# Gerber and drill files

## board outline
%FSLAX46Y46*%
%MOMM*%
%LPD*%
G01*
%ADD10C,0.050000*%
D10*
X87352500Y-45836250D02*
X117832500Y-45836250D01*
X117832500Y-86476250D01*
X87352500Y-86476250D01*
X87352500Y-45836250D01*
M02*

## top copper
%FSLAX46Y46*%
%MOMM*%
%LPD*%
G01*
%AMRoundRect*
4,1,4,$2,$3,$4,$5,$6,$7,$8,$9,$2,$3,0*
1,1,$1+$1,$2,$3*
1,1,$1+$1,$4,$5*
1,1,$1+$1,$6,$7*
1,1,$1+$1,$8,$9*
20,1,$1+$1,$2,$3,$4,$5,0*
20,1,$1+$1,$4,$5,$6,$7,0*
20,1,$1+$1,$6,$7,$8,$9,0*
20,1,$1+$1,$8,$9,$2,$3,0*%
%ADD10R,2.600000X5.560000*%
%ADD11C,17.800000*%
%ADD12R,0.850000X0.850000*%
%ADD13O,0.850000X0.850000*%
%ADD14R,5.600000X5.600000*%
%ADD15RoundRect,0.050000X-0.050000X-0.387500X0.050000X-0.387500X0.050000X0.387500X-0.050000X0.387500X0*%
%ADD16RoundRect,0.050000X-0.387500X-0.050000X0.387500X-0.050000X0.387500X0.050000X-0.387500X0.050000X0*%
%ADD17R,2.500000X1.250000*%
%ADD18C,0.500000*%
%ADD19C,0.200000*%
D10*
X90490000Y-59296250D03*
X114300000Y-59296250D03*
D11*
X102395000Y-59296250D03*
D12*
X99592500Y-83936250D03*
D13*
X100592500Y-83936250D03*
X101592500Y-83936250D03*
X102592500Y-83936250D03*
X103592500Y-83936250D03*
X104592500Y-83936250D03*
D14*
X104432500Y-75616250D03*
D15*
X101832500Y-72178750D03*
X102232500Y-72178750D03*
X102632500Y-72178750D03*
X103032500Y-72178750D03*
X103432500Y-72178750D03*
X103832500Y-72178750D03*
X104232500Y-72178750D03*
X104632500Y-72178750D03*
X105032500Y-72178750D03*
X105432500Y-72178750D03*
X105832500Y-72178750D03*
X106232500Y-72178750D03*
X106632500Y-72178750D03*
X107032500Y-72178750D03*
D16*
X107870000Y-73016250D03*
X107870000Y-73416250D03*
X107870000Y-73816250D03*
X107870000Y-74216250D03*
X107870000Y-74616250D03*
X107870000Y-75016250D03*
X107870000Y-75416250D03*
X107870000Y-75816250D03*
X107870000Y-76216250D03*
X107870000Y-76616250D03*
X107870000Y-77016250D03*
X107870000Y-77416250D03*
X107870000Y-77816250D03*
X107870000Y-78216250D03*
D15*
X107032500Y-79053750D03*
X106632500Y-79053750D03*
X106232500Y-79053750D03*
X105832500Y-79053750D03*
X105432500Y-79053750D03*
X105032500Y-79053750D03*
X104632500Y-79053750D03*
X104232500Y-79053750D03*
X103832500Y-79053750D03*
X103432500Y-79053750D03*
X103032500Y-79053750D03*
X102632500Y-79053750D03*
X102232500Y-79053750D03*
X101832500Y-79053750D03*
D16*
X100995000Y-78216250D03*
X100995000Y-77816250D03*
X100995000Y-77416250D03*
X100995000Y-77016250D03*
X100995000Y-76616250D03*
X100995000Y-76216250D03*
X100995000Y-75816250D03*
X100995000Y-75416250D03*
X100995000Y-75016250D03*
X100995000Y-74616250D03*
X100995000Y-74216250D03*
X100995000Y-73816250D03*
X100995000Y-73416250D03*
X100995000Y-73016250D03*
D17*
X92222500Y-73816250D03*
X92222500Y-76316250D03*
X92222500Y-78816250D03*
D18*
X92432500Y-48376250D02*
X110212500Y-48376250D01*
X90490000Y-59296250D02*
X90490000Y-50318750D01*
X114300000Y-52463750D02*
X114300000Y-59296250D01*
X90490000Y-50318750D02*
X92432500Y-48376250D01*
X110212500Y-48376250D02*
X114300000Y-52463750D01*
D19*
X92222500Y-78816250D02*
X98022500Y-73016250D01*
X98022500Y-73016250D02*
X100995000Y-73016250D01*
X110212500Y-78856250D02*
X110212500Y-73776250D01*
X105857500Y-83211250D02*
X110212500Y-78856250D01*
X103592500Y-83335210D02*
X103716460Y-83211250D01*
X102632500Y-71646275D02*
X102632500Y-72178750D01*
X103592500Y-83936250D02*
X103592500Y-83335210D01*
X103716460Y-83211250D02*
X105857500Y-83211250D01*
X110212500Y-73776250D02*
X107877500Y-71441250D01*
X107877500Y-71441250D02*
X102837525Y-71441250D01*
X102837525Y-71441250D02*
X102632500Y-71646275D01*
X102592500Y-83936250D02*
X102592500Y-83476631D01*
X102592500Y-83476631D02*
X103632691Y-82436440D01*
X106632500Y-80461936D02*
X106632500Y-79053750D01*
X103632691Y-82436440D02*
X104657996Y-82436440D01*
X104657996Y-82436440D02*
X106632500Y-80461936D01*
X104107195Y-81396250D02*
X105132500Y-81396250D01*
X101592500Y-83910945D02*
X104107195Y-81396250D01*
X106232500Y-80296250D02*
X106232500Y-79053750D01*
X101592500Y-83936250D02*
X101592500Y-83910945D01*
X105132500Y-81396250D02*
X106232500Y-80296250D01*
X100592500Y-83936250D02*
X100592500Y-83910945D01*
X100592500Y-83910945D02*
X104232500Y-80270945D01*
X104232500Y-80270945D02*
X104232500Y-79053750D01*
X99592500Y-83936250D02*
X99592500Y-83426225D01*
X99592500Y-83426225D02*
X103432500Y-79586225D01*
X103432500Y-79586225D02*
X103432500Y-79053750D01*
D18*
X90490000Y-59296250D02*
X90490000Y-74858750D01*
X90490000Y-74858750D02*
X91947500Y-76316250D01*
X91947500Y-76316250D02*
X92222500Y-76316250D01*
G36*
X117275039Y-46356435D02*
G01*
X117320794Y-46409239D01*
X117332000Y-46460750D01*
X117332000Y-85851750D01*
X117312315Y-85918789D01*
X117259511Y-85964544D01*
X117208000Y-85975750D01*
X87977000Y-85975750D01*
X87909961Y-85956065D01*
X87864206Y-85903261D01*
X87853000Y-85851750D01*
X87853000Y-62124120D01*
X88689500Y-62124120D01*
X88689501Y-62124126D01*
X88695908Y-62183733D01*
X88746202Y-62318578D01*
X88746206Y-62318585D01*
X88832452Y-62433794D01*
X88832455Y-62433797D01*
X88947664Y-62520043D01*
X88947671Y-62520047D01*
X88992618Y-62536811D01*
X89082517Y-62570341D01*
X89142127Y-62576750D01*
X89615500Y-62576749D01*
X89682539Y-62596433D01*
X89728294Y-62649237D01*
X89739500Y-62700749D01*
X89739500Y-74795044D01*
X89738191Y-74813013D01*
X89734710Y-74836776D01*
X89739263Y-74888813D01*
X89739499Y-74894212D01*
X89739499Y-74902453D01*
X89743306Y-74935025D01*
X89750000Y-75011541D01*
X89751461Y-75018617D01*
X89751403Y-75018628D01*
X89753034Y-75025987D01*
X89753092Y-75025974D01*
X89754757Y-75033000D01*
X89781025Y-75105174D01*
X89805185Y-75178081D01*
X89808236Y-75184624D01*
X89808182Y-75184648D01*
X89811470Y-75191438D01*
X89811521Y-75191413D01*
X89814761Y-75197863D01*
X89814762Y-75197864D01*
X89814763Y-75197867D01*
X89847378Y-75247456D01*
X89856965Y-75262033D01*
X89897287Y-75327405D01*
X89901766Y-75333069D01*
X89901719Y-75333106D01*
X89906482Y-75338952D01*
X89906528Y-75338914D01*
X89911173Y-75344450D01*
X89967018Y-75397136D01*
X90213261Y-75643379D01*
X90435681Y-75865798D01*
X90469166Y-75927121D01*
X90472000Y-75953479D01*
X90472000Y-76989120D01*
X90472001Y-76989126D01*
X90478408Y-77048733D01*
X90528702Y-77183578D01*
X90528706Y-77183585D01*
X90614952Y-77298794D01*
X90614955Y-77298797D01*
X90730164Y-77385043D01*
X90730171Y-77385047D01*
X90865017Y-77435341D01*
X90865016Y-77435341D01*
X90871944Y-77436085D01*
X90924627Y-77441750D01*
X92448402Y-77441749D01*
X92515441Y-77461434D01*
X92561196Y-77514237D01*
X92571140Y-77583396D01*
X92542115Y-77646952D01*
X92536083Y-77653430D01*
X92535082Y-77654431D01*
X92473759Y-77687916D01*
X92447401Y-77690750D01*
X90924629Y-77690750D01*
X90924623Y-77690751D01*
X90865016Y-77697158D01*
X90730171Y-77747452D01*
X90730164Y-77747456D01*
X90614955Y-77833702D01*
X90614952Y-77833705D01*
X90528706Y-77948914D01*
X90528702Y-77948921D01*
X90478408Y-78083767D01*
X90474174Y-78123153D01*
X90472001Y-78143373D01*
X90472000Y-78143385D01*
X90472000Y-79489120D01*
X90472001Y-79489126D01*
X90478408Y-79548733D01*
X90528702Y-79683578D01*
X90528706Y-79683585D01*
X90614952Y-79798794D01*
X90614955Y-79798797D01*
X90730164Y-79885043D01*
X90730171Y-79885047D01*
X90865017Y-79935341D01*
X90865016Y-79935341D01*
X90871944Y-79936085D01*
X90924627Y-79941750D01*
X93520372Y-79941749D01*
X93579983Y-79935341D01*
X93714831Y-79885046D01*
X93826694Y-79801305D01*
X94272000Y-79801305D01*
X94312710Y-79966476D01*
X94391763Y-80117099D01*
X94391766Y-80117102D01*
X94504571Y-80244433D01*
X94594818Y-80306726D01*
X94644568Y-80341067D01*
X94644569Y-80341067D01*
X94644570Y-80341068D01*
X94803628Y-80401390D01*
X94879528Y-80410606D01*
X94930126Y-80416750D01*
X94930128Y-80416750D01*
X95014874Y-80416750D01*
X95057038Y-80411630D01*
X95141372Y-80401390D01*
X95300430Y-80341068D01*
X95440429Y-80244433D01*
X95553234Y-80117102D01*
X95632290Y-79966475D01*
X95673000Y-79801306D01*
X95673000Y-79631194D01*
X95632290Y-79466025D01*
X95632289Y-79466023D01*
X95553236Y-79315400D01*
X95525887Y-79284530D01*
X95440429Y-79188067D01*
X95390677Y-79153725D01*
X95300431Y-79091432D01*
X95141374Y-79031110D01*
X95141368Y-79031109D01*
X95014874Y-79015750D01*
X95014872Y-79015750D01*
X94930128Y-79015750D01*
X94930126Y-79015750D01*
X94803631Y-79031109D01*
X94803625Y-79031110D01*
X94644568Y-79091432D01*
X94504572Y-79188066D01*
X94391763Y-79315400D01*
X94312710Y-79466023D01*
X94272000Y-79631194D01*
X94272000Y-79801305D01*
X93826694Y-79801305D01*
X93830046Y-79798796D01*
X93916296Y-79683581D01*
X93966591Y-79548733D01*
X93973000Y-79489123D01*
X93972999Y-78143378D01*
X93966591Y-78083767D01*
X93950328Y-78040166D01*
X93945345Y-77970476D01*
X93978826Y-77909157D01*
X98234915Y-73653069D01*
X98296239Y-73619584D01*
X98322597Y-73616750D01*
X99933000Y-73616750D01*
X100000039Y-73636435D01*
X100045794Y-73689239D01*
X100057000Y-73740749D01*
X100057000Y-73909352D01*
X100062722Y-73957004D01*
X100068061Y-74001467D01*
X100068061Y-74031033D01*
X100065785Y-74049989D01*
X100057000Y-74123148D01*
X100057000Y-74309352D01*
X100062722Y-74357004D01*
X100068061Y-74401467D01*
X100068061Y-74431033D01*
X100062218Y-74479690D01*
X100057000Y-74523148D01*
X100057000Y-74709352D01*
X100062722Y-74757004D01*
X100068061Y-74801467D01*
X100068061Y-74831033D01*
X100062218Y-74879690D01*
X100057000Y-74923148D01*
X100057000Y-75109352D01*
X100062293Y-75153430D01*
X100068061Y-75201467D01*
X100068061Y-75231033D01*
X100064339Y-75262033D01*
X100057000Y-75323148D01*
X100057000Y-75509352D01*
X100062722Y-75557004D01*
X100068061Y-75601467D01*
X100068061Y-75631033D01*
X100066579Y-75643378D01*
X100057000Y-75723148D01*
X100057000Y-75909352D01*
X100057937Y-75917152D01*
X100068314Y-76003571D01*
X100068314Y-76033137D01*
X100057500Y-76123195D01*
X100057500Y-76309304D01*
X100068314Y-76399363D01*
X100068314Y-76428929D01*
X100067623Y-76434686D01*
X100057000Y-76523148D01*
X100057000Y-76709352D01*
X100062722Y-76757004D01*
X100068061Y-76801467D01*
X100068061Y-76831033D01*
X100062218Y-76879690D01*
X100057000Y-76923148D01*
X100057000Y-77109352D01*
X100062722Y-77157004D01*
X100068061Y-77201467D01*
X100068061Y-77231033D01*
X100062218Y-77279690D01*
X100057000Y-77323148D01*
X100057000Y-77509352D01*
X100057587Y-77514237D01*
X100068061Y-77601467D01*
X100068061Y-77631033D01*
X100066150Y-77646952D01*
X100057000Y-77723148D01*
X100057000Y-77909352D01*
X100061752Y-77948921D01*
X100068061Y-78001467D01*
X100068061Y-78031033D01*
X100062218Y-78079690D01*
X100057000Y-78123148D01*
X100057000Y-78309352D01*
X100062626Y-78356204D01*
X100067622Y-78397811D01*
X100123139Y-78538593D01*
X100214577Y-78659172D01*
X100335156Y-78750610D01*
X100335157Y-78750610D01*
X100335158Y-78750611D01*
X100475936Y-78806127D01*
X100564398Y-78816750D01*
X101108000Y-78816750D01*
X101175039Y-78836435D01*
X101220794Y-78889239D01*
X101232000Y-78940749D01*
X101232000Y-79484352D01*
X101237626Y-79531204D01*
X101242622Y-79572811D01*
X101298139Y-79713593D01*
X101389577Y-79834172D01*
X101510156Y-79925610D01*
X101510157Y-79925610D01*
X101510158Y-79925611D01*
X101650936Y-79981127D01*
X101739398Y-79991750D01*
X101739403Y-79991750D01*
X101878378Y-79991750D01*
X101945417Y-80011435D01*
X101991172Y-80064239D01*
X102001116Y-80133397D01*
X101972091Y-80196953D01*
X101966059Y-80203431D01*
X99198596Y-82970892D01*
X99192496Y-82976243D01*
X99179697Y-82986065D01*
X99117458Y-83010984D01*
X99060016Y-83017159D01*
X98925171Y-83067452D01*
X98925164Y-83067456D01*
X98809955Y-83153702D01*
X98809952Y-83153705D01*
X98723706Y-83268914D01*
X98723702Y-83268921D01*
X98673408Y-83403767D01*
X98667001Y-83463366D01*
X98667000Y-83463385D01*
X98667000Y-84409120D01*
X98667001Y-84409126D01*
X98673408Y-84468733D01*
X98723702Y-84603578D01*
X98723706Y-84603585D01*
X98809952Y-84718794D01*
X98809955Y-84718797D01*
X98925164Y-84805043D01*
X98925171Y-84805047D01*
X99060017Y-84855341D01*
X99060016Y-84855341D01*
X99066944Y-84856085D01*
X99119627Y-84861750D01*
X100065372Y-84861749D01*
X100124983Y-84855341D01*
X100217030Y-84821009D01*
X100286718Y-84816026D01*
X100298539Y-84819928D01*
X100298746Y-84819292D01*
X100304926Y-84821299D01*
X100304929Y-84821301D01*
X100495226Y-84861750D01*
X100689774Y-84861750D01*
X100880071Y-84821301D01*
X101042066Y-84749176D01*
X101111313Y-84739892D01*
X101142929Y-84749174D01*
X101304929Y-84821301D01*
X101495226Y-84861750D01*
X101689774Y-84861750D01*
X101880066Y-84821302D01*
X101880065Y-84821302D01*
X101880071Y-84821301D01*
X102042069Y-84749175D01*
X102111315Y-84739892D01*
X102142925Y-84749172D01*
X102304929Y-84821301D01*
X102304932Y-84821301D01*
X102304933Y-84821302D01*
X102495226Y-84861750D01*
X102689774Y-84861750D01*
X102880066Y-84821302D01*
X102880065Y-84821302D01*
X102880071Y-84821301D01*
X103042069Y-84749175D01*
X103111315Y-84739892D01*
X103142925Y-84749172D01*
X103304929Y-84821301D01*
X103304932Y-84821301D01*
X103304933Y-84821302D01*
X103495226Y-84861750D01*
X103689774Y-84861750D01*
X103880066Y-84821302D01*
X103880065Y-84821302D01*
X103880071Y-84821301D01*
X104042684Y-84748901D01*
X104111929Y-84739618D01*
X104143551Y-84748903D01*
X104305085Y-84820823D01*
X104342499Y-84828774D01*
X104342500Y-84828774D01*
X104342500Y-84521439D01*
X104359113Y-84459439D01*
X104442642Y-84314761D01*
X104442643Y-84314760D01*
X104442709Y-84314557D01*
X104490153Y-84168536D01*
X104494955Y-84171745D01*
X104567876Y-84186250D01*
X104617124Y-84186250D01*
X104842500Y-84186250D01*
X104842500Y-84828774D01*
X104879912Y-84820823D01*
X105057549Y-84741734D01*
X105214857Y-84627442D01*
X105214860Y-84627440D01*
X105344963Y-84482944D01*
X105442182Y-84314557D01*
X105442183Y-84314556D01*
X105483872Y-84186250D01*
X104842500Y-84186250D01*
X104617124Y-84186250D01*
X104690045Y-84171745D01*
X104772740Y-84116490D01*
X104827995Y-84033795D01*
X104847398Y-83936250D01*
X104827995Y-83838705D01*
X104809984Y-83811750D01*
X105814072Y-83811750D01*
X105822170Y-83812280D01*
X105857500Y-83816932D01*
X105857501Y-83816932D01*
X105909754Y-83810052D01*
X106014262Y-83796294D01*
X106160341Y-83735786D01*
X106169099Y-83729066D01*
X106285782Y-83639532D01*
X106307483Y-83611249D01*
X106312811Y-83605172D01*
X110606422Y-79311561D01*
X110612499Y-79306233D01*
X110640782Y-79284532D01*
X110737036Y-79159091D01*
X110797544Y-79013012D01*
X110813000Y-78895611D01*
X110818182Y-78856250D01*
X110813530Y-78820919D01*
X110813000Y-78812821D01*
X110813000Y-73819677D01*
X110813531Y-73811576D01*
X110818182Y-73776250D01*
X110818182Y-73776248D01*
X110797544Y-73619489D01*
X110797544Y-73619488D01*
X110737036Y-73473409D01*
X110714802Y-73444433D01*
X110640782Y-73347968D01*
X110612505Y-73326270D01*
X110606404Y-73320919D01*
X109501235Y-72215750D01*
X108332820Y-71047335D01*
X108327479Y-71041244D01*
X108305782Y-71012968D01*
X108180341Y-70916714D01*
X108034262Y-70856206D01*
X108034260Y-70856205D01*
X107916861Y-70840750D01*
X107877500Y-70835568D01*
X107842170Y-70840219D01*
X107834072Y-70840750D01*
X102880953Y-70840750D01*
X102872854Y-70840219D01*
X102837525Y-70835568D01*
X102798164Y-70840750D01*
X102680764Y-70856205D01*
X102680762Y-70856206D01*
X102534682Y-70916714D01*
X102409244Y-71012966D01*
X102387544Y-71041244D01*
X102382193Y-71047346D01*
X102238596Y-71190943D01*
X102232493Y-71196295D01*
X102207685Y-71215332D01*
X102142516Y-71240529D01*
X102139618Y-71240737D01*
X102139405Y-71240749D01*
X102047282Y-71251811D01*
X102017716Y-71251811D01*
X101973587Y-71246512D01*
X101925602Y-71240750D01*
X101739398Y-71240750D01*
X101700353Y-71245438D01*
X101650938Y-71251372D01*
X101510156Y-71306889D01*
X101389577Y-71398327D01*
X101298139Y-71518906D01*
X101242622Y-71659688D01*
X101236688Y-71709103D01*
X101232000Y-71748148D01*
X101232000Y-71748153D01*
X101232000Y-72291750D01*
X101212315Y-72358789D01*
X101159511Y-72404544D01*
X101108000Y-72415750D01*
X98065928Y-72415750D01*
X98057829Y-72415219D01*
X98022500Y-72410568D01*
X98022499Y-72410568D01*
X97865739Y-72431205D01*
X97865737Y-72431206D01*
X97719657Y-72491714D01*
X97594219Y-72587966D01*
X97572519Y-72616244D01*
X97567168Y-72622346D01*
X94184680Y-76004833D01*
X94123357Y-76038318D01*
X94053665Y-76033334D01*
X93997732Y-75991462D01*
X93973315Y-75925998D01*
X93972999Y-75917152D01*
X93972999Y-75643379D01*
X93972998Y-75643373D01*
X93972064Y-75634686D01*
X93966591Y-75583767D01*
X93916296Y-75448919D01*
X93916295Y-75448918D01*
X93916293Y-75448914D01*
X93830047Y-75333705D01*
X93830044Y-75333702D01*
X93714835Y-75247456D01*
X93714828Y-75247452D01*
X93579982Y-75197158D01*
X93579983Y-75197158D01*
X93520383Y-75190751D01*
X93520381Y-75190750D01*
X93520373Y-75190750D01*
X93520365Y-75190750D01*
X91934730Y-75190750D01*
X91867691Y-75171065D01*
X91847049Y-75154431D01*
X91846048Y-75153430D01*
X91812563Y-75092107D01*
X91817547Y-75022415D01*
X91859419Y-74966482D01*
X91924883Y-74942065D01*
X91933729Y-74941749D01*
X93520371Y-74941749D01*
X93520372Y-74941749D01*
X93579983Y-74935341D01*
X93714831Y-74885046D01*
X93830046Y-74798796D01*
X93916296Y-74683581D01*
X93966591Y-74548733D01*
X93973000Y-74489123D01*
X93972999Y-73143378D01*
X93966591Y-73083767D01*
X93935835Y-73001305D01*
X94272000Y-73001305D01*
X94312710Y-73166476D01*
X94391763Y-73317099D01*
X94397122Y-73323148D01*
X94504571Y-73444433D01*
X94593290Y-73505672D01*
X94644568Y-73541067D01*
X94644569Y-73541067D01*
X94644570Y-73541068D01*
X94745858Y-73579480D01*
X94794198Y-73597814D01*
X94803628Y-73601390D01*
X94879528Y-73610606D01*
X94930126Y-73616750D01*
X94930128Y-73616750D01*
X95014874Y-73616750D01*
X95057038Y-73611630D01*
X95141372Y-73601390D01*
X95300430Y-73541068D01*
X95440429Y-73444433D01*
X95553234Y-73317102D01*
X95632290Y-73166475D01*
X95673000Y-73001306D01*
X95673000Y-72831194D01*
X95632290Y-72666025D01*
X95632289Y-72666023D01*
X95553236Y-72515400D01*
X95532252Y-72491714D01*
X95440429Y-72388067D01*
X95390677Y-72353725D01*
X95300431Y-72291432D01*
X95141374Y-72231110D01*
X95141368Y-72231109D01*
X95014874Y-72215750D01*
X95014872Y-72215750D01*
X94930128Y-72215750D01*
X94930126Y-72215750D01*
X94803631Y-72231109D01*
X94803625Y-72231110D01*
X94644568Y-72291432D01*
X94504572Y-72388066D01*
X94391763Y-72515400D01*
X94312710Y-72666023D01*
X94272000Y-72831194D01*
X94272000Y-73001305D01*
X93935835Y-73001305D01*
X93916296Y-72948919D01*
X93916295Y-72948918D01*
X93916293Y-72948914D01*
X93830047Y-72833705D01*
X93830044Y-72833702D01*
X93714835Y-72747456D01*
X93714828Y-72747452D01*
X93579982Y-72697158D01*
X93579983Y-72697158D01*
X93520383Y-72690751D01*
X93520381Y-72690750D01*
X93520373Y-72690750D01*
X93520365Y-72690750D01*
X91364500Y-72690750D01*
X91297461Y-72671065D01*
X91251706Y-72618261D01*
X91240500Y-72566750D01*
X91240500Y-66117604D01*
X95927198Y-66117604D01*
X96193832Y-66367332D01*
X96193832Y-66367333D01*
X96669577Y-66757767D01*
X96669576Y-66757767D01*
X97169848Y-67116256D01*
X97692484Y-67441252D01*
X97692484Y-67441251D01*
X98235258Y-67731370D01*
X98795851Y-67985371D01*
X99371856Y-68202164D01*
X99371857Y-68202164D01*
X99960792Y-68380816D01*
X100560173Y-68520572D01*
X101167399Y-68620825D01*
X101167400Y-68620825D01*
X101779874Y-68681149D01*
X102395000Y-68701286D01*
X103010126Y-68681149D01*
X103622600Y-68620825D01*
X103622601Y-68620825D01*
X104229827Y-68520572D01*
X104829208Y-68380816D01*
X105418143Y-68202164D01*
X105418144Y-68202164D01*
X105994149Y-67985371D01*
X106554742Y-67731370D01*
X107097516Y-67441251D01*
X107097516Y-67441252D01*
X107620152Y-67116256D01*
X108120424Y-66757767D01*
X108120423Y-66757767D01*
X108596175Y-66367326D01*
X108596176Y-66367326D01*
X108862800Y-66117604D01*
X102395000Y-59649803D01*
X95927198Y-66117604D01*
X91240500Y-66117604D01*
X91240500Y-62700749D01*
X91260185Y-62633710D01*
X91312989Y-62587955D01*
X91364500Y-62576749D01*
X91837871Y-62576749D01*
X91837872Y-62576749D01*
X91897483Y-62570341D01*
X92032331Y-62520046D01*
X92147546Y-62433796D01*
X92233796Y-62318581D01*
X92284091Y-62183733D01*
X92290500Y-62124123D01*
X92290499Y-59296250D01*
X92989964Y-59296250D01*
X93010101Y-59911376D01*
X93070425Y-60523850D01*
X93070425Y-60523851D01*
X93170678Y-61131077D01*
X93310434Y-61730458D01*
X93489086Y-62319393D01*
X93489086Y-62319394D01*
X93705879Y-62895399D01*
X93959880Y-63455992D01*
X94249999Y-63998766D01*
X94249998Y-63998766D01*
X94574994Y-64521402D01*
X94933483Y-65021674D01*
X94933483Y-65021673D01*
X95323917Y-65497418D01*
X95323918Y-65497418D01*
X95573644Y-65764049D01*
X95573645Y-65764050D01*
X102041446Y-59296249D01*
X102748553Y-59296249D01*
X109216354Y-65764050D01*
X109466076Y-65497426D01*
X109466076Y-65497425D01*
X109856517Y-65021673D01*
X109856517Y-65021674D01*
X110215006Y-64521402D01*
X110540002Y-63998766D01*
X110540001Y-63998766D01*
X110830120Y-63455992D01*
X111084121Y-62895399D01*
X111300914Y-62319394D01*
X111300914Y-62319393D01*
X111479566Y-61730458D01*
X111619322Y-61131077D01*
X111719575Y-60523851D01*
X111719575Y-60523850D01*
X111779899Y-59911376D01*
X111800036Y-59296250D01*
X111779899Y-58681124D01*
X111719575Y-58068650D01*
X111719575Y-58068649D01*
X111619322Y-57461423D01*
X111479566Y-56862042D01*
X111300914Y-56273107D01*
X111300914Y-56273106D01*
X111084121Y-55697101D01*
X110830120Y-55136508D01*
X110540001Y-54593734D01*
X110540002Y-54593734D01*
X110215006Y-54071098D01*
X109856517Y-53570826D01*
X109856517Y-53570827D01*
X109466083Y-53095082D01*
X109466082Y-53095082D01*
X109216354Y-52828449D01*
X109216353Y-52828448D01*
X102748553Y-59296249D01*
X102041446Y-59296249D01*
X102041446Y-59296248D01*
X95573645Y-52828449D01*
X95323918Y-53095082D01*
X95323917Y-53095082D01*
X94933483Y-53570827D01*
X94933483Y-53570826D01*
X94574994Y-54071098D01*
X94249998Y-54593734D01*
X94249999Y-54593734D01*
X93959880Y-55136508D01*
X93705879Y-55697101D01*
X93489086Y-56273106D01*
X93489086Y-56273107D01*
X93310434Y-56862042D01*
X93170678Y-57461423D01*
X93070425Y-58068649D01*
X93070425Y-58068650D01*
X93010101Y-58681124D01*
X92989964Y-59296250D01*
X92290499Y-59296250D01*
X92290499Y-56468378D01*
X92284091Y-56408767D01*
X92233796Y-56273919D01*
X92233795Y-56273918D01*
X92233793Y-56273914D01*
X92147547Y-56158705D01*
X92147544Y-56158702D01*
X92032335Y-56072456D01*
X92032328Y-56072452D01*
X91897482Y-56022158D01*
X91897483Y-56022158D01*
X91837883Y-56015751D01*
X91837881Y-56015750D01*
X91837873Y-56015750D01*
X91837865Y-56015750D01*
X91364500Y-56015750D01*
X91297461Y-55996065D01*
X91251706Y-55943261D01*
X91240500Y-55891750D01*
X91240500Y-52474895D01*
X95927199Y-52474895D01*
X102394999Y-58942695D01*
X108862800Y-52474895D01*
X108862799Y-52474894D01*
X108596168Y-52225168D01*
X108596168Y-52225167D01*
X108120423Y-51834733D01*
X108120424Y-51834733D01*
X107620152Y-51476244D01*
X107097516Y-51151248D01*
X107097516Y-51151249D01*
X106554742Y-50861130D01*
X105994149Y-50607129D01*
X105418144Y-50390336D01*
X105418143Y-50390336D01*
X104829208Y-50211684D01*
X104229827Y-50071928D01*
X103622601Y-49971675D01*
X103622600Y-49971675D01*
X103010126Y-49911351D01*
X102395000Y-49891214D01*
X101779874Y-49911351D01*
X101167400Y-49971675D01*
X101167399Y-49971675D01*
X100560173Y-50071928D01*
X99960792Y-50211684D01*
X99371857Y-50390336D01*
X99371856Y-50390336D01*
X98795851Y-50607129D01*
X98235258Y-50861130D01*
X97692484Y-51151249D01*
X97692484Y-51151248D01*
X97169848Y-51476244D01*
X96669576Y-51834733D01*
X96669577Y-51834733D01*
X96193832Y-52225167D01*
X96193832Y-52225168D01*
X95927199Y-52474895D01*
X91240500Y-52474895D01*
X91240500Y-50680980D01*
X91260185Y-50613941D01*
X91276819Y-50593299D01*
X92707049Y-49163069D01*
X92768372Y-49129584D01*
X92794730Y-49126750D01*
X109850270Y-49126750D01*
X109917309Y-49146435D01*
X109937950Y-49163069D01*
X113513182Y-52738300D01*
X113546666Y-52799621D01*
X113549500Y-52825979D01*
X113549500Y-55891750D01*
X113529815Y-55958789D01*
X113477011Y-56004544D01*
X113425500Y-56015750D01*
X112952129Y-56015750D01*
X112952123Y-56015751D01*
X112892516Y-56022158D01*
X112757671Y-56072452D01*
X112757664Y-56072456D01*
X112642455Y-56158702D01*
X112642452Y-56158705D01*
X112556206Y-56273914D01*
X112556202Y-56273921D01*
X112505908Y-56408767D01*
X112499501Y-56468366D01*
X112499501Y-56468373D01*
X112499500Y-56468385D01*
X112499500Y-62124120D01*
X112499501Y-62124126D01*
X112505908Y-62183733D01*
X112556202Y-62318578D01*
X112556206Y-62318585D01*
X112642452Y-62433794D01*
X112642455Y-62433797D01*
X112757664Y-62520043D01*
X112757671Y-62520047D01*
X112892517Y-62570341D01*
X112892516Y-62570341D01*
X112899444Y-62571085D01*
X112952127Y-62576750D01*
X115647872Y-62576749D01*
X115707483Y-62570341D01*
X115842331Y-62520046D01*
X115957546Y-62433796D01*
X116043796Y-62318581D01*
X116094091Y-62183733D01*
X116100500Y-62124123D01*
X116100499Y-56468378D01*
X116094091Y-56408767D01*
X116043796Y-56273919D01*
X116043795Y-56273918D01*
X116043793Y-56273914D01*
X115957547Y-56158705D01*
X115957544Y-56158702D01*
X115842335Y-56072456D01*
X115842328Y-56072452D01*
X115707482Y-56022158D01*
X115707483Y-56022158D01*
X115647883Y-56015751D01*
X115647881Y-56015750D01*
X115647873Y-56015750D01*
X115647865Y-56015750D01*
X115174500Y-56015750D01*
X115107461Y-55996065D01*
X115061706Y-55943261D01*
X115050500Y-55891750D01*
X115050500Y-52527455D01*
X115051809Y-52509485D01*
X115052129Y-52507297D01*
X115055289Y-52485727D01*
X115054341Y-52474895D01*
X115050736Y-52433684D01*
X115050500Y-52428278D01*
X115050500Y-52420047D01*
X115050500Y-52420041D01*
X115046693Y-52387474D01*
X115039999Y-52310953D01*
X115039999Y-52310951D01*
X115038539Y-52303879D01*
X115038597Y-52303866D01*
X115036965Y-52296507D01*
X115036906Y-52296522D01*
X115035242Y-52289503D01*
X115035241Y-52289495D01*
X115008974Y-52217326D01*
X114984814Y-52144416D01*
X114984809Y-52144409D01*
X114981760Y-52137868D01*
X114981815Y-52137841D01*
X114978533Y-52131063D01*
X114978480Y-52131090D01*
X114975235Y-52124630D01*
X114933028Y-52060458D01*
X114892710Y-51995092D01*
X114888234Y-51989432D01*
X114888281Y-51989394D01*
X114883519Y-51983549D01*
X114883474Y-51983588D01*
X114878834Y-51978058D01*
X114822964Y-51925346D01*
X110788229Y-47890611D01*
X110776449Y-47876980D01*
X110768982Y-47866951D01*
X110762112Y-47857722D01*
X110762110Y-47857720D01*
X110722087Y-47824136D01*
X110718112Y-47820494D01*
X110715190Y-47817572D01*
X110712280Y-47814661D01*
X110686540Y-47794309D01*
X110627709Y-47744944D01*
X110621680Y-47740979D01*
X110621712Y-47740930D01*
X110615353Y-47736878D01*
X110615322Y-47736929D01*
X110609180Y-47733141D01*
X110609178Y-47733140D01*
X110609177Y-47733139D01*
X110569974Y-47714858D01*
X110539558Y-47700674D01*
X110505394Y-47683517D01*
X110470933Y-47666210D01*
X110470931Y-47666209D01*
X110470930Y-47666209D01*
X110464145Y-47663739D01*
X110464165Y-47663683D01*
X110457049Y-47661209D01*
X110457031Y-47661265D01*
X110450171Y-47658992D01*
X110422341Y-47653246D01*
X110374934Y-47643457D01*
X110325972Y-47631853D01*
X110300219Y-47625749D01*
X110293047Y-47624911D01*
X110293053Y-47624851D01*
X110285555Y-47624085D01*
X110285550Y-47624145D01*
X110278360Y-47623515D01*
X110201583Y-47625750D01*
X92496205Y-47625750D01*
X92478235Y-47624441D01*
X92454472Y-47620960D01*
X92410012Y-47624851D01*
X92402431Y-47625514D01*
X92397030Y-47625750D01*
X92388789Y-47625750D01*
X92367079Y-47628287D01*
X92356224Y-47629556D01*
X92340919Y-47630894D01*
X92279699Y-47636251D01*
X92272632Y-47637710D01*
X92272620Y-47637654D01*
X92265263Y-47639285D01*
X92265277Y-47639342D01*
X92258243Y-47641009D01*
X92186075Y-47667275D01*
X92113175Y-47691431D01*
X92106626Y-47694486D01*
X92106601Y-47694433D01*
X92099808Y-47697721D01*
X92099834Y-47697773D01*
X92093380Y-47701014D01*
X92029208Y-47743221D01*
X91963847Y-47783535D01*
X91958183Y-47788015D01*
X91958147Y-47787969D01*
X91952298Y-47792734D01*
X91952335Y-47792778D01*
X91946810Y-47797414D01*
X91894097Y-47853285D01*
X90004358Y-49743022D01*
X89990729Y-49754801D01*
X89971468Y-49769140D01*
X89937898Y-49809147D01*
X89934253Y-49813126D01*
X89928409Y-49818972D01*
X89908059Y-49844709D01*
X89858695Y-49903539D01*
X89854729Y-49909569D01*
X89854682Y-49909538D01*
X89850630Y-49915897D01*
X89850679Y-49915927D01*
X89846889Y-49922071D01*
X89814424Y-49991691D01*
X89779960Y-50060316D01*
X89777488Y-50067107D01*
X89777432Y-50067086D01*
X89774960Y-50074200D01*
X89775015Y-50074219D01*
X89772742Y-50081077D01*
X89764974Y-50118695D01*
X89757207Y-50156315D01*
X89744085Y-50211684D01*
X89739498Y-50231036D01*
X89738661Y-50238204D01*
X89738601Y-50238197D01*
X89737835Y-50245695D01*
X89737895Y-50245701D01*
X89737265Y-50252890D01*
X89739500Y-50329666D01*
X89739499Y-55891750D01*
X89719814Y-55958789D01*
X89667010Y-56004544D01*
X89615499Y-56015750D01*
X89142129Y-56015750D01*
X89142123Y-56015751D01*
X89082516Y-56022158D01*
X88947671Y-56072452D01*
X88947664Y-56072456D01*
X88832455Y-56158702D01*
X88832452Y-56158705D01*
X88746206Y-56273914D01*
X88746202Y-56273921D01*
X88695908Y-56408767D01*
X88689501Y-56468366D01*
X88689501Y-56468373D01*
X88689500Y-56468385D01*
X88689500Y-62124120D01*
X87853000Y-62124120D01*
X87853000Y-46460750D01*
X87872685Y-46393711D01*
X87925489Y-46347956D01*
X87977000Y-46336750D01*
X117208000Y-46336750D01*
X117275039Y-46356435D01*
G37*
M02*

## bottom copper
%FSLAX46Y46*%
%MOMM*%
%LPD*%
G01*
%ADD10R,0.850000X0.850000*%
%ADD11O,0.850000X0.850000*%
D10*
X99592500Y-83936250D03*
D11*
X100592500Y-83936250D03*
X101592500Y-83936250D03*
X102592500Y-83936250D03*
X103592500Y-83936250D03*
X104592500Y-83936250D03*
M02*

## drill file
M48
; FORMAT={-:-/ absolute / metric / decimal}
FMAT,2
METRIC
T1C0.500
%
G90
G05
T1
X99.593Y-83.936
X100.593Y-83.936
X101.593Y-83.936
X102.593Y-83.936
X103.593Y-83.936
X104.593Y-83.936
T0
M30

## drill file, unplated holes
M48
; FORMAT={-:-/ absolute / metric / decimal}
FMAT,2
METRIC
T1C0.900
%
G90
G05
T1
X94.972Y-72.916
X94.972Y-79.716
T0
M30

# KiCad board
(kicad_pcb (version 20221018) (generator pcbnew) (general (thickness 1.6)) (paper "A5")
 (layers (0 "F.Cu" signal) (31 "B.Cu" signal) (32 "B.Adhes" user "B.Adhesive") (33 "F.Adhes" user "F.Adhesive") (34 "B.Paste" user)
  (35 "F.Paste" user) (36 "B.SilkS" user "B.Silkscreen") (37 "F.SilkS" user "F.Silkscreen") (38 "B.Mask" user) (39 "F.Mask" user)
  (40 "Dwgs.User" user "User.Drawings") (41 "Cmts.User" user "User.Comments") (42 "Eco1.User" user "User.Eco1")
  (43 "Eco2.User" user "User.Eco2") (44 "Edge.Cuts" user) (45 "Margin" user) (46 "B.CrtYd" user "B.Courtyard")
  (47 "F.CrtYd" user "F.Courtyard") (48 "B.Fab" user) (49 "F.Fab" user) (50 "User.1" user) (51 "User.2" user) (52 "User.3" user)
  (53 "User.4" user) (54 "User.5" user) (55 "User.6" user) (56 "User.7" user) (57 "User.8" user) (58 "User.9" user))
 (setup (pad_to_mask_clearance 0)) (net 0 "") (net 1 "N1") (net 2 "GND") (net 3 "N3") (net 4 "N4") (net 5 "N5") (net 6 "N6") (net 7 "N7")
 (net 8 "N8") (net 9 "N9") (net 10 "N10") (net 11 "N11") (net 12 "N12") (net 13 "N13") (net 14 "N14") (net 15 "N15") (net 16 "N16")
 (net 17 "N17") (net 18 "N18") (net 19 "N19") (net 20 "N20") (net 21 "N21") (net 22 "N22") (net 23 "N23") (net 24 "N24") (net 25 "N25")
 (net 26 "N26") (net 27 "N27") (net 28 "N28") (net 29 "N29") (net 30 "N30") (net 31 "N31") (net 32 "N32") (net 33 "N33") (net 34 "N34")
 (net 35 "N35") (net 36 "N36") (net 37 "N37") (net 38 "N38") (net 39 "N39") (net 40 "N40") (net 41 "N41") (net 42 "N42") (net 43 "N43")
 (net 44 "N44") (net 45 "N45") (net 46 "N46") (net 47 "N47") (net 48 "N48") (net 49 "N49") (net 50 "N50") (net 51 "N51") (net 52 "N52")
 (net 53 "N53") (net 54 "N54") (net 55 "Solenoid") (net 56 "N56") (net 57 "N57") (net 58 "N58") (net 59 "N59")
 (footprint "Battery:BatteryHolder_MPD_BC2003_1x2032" (layer "F.Cu") (at 102.395 59.29625)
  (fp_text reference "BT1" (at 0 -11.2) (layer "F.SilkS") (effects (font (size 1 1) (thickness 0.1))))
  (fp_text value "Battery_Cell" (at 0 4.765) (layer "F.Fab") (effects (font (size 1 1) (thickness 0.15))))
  (pad "1" smd rect (at -11.905 0) (size 2.6 5.56) (layers "F.Cu" "F.Paste" "F.Mask") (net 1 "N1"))
  (pad "1" smd rect (at 11.905 0) (size 2.6 5.56) (layers "F.Cu" "F.Paste" "F.Mask") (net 1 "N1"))
  (pad "2" smd circle (at 0 0) (size 17.8 17.8) (layers "F.Cu" "F.Mask") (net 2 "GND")))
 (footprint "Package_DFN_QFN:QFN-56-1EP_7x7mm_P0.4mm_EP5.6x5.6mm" (layer "F.Cu") (at 104.4325 75.61625)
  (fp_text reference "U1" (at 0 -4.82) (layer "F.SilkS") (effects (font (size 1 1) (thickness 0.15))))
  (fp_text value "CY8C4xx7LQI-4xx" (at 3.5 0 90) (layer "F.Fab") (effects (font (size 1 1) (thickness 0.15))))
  (pad "" smd roundrect (at -2.1 -2.1) (size 1.13 1.13) (layers "F.Paste") (roundrect_rratio 0.2212389381))
  (pad "" smd roundrect (at -2.1 -0.7) (size 1.13 1.13) (layers "F.Paste") (roundrect_rratio 0.2212389381))
  (pad "" smd roundrect (at -2.1 0.7) (size 1.13 1.13) (layers "F.Paste") (roundrect_rratio 0.2212389381))
  (pad "" smd roundrect (at -2.1 2.1) (size 1.13 1.13) (layers "F.Paste") (roundrect_rratio 0.2212389381))
  (pad "" smd roundrect (at -0.7 -2.1) (size 1.13 1.13) (layers "F.Paste") (roundrect_rratio 0.2212389381))
  (pad "" smd roundrect (at -0.7 -0.7) (size 1.13 1.13) (layers "F.Paste") (roundrect_rratio 0.2212389381))
  (pad "" smd roundrect (at -0.7 0.7) (size 1.13 1.13) (layers "F.Paste") (roundrect_rratio 0.2212389381))
  (pad "" smd roundrect (at -0.7 2.1) (size 1.13 1.13) (layers "F.Paste") (roundrect_rratio 0.2212389381))
  (pad "" smd roundrect (at 0.7 -2.1) (size 1.13 1.13) (layers "F.Paste") (roundrect_rratio 0.2212389381))
  (pad "" smd roundrect (at 0.7 -0.7) (size 1.13 1.13) (layers "F.Paste") (roundrect_rratio 0.2212389381))
  (pad "" smd roundrect (at 0.7 0.7) (size 1.13 1.13) (layers "F.Paste") (roundrect_rratio 0.2212389381))
  (pad "" smd roundrect (at 0.7 2.1) (size 1.13 1.13) (layers "F.Paste") (roundrect_rratio 0.2212389381))
  (pad "" smd roundrect (at 2.1 -2.1) (size 1.13 1.13) (layers "F.Paste") (roundrect_rratio 0.2212389381))
  (pad "" smd roundrect (at 2.1 -0.7) (size 1.13 1.13) (layers "F.Paste") (roundrect_rratio 0.2212389381))
  (pad "" smd roundrect (at 2.1 0.7) (size 1.13 1.13) (layers "F.Paste") (roundrect_rratio 0.2212389381))
  (pad "" smd roundrect (at 2.1 2.1) (size 1.13 1.13) (layers "F.Paste") (roundrect_rratio 0.2212389381))
  (pad "1" smd roundrect (at -3.4375 -2.6) (size 0.875 0.2) (layers "F.Cu" "F.Paste" "F.Mask") (roundrect_rratio 0.25) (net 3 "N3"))
  (pad "2" smd roundrect (at -3.4375 -2.2) (size 0.875 0.2) (layers "F.Cu" "F.Paste" "F.Mask") (roundrect_rratio 0.25) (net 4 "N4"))
  (pad "3" smd roundrect (at -3.4375 -1.8) (size 0.875 0.2) (layers "F.Cu" "F.Paste" "F.Mask") (roundrect_rratio 0.25) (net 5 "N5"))
  (pad "4" smd roundrect (at -3.4375 -1.4) (size 0.875 0.2) (layers "F.Cu" "F.Paste" "F.Mask") (roundrect_rratio 0.25) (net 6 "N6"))
  (pad "5" smd roundrect (at -3.4375 -1) (size 0.875 0.2) (layers "F.Cu" "F.Paste" "F.Mask") (roundrect_rratio 0.25) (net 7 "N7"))
  (pad "6" smd roundrect (at -3.4375 -0.6) (size 0.875 0.2) (layers "F.Cu" "F.Paste" "F.Mask") (roundrect_rratio 0.25) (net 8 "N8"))
  (pad "7" smd roundrect (at -3.4375 -0.2) (size 0.875 0.2) (layers "F.Cu" "F.Paste" "F.Mask") (roundrect_rratio 0.25) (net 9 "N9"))
  (pad "8" smd roundrect (at -3.4375 0.2) (size 0.875 0.2) (layers "F.Cu" "F.Paste" "F.Mask") (roundrect_rratio 0.25) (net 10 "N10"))
  (pad "9" smd roundrect (at -3.4375 0.6) (size 0.875 0.2) (layers "F.Cu" "F.Paste" "F.Mask") (roundrect_rratio 0.25) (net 2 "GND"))
  (pad "10" smd roundrect (at -3.4375 1) (size 0.875 0.2) (layers "F.Cu" "F.Paste" "F.Mask") (roundrect_rratio 0.25) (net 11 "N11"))
  (pad "11" smd roundrect (at -3.4375 1.4) (size 0.875 0.2) (layers "F.Cu" "F.Paste" "F.Mask") (roundrect_rratio 0.25) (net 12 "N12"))
  (pad "12" smd roundrect (at -3.4375 1.8) (size 0.875 0.2) (layers "F.Cu" "F.Paste" "F.Mask") (roundrect_rratio 0.25) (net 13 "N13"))
  (pad "13" smd roundrect (at -3.4375 2.2) (size 0.875 0.2) (layers "F.Cu" "F.Paste" "F.Mask") (roundrect_rratio 0.25) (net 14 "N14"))
  (pad "14" smd roundrect (at -3.4375 2.6) (size 0.875 0.2) (layers "F.Cu" "F.Paste" "F.Mask") (roundrect_rratio 0.25) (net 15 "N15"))
  (pad "15" smd roundrect (at -2.6 3.4375) (size 0.2 0.875) (layers "F.Cu" "F.Paste" "F.Mask") (roundrect_rratio 0.25) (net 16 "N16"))
  (pad "16" smd roundrect (at -2.2 3.4375) (size 0.2 0.875) (layers "F.Cu" "F.Paste" "F.Mask") (roundrect_rratio 0.25) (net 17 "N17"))
  (pad "17" smd roundrect (at -1.8 3.4375) (size 0.2 0.875) (layers "F.Cu" "F.Paste" "F.Mask") (roundrect_rratio 0.25) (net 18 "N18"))
  (pad "18" smd roundrect (at -1.4 3.4375) (size 0.2 0.875) (layers "F.Cu" "F.Paste" "F.Mask") (roundrect_rratio 0.25) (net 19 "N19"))
  (pad "19" smd roundrect (at -1 3.4375) (size 0.2 0.875) (layers "F.Cu" "F.Paste" "F.Mask") (roundrect_rratio 0.25) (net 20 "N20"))
  (pad "20" smd roundrect (at -0.6 3.4375) (size 0.2 0.875) (layers "F.Cu" "F.Paste" "F.Mask") (roundrect_rratio 0.25) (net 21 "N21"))
  (pad "21" smd roundrect (at -0.2 3.4375) (size 0.2 0.875) (layers "F.Cu" "F.Paste" "F.Mask") (roundrect_rratio 0.25) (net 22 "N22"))
  (pad "22" smd roundrect (at 0.2 3.4375) (size 0.2 0.875) (layers "F.Cu" "F.Paste" "F.Mask") (roundrect_rratio 0.25) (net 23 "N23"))
  (pad "23" smd roundrect (at 0.6 3.4375) (size 0.2 0.875) (layers "F.Cu" "F.Paste" "F.Mask") (roundrect_rratio 0.25) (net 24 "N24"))
  (pad "24" smd roundrect (at 1 3.4375) (size 0.2 0.875) (layers "F.Cu" "F.Paste" "F.Mask") (roundrect_rratio 0.25) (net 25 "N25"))
  (pad "25" smd roundrect (at 1.4 3.4375) (size 0.2 0.875) (layers "F.Cu" "F.Paste" "F.Mask") (roundrect_rratio 0.25) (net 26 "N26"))
  (pad "26" smd roundrect (at 1.8 3.4375) (size 0.2 0.875) (layers "F.Cu" "F.Paste" "F.Mask") (roundrect_rratio 0.25) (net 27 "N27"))
  (pad "27" smd roundrect (at 2.2 3.4375) (size 0.2 0.875) (layers "F.Cu" "F.Paste" "F.Mask") (roundrect_rratio 0.25) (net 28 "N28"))
  (pad "28" smd roundrect (at 2.6 3.4375) (size 0.2 0.875) (layers "F.Cu" "F.Paste" "F.Mask") (roundrect_rratio 0.25) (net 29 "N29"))
  (pad "29" smd roundrect (at 3.4375 2.6) (size 0.875 0.2) (layers "F.Cu" "F.Paste" "F.Mask") (roundrect_rratio 0.25) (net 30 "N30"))
  (pad "30" smd roundrect (at 3.4375 2.2) (size 0.875 0.2) (layers "F.Cu" "F.Paste" "F.Mask") (roundrect_rratio 0.25) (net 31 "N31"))
  (pad "31" smd roundrect (at 3.4375 1.8) (size 0.875 0.2) (layers "F.Cu" "F.Paste" "F.Mask") (roundrect_rratio 0.25) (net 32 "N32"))
  (pad "32" smd roundrect (at 3.4375 1.4) (size 0.875 0.2) (layers "F.Cu" "F.Paste" "F.Mask") (roundrect_rratio 0.25) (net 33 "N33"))
  (pad "33" smd roundrect (at 3.4375 1) (size 0.875 0.2) (layers "F.Cu" "F.Paste" "F.Mask") (roundrect_rratio 0.25) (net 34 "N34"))
  (pad "34" smd roundrect (at 3.4375 0.6) (size 0.875 0.2) (layers "F.Cu" "F.Paste" "F.Mask") (roundrect_rratio 0.25) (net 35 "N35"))
  (pad "35" smd roundrect (at 3.4375 0.2) (size 0.875 0.2) (layers "F.Cu" "F.Paste" "F.Mask") (roundrect_rratio 0.25) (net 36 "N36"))
  (pad "36" smd roundrect (at 3.4375 -0.2) (size 0.875 0.2) (layers "F.Cu" "F.Paste" "F.Mask") (roundrect_rratio 0.25) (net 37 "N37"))
  (pad "37" smd roundrect (at 3.4375 -0.6) (size 0.875 0.2) (layers "F.Cu" "F.Paste" "F.Mask") (roundrect_rratio 0.25) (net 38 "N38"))
  (pad "38" smd roundrect (at 3.4375 -1) (size 0.875 0.2) (layers "F.Cu" "F.Paste" "F.Mask") (roundrect_rratio 0.25) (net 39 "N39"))
  (pad "39" smd roundrect (at 3.4375 -1.4) (size 0.875 0.2) (layers "F.Cu" "F.Paste" "F.Mask") (roundrect_rratio 0.25) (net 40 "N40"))
  (pad "40" smd roundrect (at 3.4375 -1.8) (size 0.875 0.2) (layers "F.Cu" "F.Paste" "F.Mask") (roundrect_rratio 0.25) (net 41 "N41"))
  (pad "41" smd roundrect (at 3.4375 -2.2) (size 0.875 0.2) (layers "F.Cu" "F.Paste" "F.Mask") (roundrect_rratio 0.25) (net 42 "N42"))
  (pad "42" smd roundrect (at 3.4375 -2.6) (size 0.875 0.2) (layers "F.Cu" "F.Paste" "F.Mask") (roundrect_rratio 0.25) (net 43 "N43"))
  (pad "43" smd roundrect (at 2.6 -3.4375) (size 0.2 0.875) (layers "F.Cu" "F.Paste" "F.Mask") (roundrect_rratio 0.25) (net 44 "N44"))
  (pad "44" smd roundrect (at 2.2 -3.4375) (size 0.2 0.875) (layers "F.Cu" "F.Paste" "F.Mask") (roundrect_rratio 0.25) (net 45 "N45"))
  (pad "45" smd roundrect (at 1.8 -3.4375) (size 0.2 0.875) (layers "F.Cu" "F.Paste" "F.Mask") (roundrect_rratio 0.25) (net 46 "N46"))
  (pad "46" smd roundrect (at 1.4 -3.4375) (size 0.2 0.875) (layers "F.Cu" "F.Paste" "F.Mask") (roundrect_rratio 0.25) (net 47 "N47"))
  (pad "47" smd roundrect (at 1 -3.4375) (size 0.2 0.875) (layers "F.Cu" "F.Paste" "F.Mask") (roundrect_rratio 0.25) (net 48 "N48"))
  (pad "48" smd roundrect (at 0.6 -3.4375) (size 0.2 0.875) (layers "F.Cu" "F.Paste" "F.Mask") (roundrect_rratio 0.25) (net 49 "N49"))
  (pad "49" smd roundrect (at 0.2 -3.4375) (size 0.2 0.875) (layers "F.Cu" "F.Paste" "F.Mask") (roundrect_rratio 0.25) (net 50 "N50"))
  (pad "50" smd roundrect (at -0.2 -3.4375) (size 0.2 0.875) (layers "F.Cu" "F.Paste" "F.Mask") (roundrect_rratio 0.25) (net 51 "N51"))
  (pad "51" smd roundrect (at -0.6 -3.4375) (size 0.2 0.875) (layers "F.Cu" "F.Paste" "F.Mask") (roundrect_rratio 0.25) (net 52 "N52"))
  (pad "52" smd roundrect (at -1 -3.4375) (size 0.2 0.875) (layers "F.Cu" "F.Paste" "F.Mask") (roundrect_rratio 0.25) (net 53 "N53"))
  (pad "53" smd roundrect (at -1.4 -3.4375) (size 0.2 0.875) (layers "F.Cu" "F.Paste" "F.Mask") (roundrect_rratio 0.25) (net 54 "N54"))
  (pad "54" smd roundrect (at -1.8 -3.4375) (size 0.2 0.875) (layers "F.Cu" "F.Paste" "F.Mask") (roundrect_rratio 0.25) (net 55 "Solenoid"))
  (pad "55" smd roundrect (at -2.2 -3.4375) (size 0.2 0.875) (layers "F.Cu" "F.Paste" "F.Mask") (roundrect_rratio 0.25) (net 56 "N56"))
  (pad "56" smd roundrect (at -2.6 -3.4375) (size 0.2 0.875) (layers "F.Cu" "F.Paste" "F.Mask") (roundrect_rratio 0.25) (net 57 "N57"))
  (pad "57" smd rect (at 0 0) (size 5.6 5.6) (layers "F.Cu" "F.Mask") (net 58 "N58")))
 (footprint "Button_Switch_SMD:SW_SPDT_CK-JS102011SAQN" (layer "F.Cu") (at 94.9725 76.31625 90)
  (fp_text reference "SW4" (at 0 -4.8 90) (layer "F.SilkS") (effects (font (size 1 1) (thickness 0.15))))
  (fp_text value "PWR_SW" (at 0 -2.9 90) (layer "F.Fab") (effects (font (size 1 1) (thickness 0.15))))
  (pad "" np_thru_hole circle (at -3.4 0 90) (size 0.9 0.9) (drill 0.9) (layers "*.Cu" "*.Mask"))
  (pad "" np_thru_hole circle (at 3.4 0 90) (size 0.9 0.9) (drill 0.9) (layers "*.Cu" "*.Mask"))
  (pad "1" smd rect (at -2.5 -2.75 90) (size 1.25 2.5) (layers "F.Cu" "F.Paste" "F.Mask") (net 3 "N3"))
  (pad "2" smd rect (at 0 -2.75 90) (size 1.25 2.5) (layers "F.Cu" "F.Paste" "F.Mask") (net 1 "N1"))
  (pad "3" smd rect (at 2.5 -2.75 90) (size 1.25 2.5) (layers "F.Cu" "F.Paste" "F.Mask") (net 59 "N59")))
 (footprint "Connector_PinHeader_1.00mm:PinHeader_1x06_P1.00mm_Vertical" (layer "F.Cu") (at 99.5925 83.93625 90)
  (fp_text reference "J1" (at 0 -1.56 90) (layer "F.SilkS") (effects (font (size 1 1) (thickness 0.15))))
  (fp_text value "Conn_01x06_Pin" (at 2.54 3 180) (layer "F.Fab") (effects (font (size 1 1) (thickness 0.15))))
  (pad "1" thru_hole rect (at 0 0 90) (size 0.85 0.85) (drill 0.5) (layers "*.Cu" "*.Mask") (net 20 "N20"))
  (pad "2" thru_hole oval (at 0 1 90) (size 0.85 0.85) (drill 0.5) (layers "*.Cu" "*.Mask") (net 22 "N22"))
  (pad "3" thru_hole oval (at 0 2 90) (size 0.85 0.85) (drill 0.5) (layers "*.Cu" "*.Mask") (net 27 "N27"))
  (pad "4" thru_hole oval (at 0 3 90) (size 0.85 0.85) (drill 0.5) (layers "*.Cu" "*.Mask") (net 28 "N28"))
  (pad "5" thru_hole oval (at 0 4 90) (size 0.85 0.85) (drill 0.5) (layers "*.Cu" "*.Mask") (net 55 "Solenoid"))
  (pad "6" thru_hole oval (at 0 5 90) (size 0.85 0.85) (drill 0.5) (layers "*.Cu" "*.Mask") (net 2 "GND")))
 (gr_rect (start 87.3525 45.83625) (end 117.8325 86.47625) (stroke (width 0.05) (type default)) (fill none) (layer "Edge.Cuts"))
 (segment (start 92.2225 78.81625) (end 98.0225 73.01625) (width 0.2) (layer "F.Cu") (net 3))
 (segment (start 98.0225 73.01625) (end 100.995 73.01625) (width 0.2) (layer "F.Cu") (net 3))
 (segment (start 90.49 59.29625) (end 90.49 50.31875) (width 0.5) (layer "F.Cu") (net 1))
 (segment (start 90.49 74.85875) (end 91.9475 76.31625) (width 0.5) (layer "F.Cu") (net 1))
 (segment (start 92.4325 48.37625) (end 110.2125 48.37625) (width 0.5) (layer "F.Cu") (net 1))
 (segment (start 114.3 52.46375) (end 114.3 59.29625) (width 0.5) (layer "F.Cu") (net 1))
 (segment (start 90.49 59.29625) (end 90.49 74.85875) (width 0.5) (layer "F.Cu") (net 1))
 (segment (start 91.9475 76.31625) (end 92.2225 76.31625) (width 0.5) (layer "F.Cu") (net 1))
 (segment (start 110.2125 48.37625) (end 114.3 52.46375) (width 0.5) (layer "F.Cu") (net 1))
 (segment (start 90.49 50.31875) (end 92.4325 48.37625) (width 0.5) (layer "F.Cu") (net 1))
 (segment (start 103.4325 79.586225) (end 103.4325 79.05375) (width 0.2) (layer "F.Cu") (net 20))
 (segment (start 99.5925 83.93625) (end 99.5925 83.426225) (width 0.2) (layer "F.Cu") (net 20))
 (segment (start 99.5925 83.426225) (end 103.4325 79.586225) (width 0.2) (layer "F.Cu") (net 20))
 (segment (start 104.2325 80.270945) (end 104.2325 79.05375) (width 0.2) (layer "F.Cu") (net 22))
 (segment (start 100.5925 83.93625) (end 100.5925 83.910945) (width 0.2) (layer "F.Cu") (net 22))
 (segment (start 100.5925 83.910945) (end 104.2325 80.270945) (width 0.2) (layer "F.Cu") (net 22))
 (segment (start 105.1325 81.39625) (end 106.2325 80.29625) (width 0.2) (layer "F.Cu") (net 27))
 (segment (start 104.107195 81.39625) (end 105.1325 81.39625) (width 0.2) (layer "F.Cu") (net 27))
 (segment (start 101.5925 83.93625) (end 101.5925 83.910945) (width 0.2) (layer "F.Cu") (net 27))
 (segment (start 106.2325 80.29625) (end 106.2325 79.05375) (width 0.2) (layer "F.Cu") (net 27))
 (segment (start 101.5925 83.910945) (end 104.107195 81.39625) (width 0.2) (layer "F.Cu") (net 27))
 (segment (start 102.5925 83.93625) (end 102.5925 83.476631) (width 0.2) (layer "F.Cu") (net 28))
 (segment (start 103.632691 82.43644) (end 104.657996 82.43644) (width 0.2) (layer "F.Cu") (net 28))
 (segment (start 102.5925 83.476631) (end 103.632691 82.43644) (width 0.2) (layer "F.Cu") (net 28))
 (segment (start 106.6325 80.461936) (end 106.6325 79.05375) (width 0.2) (layer "F.Cu") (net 28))
 (segment (start 104.657996 82.43644) (end 106.6325 80.461936) (width 0.2) (layer "F.Cu") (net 28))
 (segment (start 110.2125 78.85625) (end 110.2125 73.77625) (width 0.2) (layer "F.Cu") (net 55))
 (segment (start 107.8775 71.44125) (end 102.837525 71.44125) (width 0.2) (layer "F.Cu") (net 55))
 (segment (start 102.837525 71.44125) (end 102.6325 71.646275) (width 0.2) (layer "F.Cu") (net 55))
 (segment (start 103.5925 83.93625) (end 103.5925 83.33521) (width 0.2) (layer "F.Cu") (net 55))
 (segment (start 103.71646 83.21125) (end 105.8575 83.21125) (width 0.2) (layer "F.Cu") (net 55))
 (segment (start 102.6325 71.646275) (end 102.6325 72.17875) (width 0.2) (layer "F.Cu") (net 55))
 (segment (start 103.5925 83.33521) (end 103.71646 83.21125) (width 0.2) (layer "F.Cu") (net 55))
 (segment (start 110.2125 73.77625) (end 107.8775 71.44125) (width 0.2) (layer "F.Cu") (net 55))
 (segment (start 105.8575 83.21125) (end 110.2125 78.85625) (width 0.2) (layer "F.Cu") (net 55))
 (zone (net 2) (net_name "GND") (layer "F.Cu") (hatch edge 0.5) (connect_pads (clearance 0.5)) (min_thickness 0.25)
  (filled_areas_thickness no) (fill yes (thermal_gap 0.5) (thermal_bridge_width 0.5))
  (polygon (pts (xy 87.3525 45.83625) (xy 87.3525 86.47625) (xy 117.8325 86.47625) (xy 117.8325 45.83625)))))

